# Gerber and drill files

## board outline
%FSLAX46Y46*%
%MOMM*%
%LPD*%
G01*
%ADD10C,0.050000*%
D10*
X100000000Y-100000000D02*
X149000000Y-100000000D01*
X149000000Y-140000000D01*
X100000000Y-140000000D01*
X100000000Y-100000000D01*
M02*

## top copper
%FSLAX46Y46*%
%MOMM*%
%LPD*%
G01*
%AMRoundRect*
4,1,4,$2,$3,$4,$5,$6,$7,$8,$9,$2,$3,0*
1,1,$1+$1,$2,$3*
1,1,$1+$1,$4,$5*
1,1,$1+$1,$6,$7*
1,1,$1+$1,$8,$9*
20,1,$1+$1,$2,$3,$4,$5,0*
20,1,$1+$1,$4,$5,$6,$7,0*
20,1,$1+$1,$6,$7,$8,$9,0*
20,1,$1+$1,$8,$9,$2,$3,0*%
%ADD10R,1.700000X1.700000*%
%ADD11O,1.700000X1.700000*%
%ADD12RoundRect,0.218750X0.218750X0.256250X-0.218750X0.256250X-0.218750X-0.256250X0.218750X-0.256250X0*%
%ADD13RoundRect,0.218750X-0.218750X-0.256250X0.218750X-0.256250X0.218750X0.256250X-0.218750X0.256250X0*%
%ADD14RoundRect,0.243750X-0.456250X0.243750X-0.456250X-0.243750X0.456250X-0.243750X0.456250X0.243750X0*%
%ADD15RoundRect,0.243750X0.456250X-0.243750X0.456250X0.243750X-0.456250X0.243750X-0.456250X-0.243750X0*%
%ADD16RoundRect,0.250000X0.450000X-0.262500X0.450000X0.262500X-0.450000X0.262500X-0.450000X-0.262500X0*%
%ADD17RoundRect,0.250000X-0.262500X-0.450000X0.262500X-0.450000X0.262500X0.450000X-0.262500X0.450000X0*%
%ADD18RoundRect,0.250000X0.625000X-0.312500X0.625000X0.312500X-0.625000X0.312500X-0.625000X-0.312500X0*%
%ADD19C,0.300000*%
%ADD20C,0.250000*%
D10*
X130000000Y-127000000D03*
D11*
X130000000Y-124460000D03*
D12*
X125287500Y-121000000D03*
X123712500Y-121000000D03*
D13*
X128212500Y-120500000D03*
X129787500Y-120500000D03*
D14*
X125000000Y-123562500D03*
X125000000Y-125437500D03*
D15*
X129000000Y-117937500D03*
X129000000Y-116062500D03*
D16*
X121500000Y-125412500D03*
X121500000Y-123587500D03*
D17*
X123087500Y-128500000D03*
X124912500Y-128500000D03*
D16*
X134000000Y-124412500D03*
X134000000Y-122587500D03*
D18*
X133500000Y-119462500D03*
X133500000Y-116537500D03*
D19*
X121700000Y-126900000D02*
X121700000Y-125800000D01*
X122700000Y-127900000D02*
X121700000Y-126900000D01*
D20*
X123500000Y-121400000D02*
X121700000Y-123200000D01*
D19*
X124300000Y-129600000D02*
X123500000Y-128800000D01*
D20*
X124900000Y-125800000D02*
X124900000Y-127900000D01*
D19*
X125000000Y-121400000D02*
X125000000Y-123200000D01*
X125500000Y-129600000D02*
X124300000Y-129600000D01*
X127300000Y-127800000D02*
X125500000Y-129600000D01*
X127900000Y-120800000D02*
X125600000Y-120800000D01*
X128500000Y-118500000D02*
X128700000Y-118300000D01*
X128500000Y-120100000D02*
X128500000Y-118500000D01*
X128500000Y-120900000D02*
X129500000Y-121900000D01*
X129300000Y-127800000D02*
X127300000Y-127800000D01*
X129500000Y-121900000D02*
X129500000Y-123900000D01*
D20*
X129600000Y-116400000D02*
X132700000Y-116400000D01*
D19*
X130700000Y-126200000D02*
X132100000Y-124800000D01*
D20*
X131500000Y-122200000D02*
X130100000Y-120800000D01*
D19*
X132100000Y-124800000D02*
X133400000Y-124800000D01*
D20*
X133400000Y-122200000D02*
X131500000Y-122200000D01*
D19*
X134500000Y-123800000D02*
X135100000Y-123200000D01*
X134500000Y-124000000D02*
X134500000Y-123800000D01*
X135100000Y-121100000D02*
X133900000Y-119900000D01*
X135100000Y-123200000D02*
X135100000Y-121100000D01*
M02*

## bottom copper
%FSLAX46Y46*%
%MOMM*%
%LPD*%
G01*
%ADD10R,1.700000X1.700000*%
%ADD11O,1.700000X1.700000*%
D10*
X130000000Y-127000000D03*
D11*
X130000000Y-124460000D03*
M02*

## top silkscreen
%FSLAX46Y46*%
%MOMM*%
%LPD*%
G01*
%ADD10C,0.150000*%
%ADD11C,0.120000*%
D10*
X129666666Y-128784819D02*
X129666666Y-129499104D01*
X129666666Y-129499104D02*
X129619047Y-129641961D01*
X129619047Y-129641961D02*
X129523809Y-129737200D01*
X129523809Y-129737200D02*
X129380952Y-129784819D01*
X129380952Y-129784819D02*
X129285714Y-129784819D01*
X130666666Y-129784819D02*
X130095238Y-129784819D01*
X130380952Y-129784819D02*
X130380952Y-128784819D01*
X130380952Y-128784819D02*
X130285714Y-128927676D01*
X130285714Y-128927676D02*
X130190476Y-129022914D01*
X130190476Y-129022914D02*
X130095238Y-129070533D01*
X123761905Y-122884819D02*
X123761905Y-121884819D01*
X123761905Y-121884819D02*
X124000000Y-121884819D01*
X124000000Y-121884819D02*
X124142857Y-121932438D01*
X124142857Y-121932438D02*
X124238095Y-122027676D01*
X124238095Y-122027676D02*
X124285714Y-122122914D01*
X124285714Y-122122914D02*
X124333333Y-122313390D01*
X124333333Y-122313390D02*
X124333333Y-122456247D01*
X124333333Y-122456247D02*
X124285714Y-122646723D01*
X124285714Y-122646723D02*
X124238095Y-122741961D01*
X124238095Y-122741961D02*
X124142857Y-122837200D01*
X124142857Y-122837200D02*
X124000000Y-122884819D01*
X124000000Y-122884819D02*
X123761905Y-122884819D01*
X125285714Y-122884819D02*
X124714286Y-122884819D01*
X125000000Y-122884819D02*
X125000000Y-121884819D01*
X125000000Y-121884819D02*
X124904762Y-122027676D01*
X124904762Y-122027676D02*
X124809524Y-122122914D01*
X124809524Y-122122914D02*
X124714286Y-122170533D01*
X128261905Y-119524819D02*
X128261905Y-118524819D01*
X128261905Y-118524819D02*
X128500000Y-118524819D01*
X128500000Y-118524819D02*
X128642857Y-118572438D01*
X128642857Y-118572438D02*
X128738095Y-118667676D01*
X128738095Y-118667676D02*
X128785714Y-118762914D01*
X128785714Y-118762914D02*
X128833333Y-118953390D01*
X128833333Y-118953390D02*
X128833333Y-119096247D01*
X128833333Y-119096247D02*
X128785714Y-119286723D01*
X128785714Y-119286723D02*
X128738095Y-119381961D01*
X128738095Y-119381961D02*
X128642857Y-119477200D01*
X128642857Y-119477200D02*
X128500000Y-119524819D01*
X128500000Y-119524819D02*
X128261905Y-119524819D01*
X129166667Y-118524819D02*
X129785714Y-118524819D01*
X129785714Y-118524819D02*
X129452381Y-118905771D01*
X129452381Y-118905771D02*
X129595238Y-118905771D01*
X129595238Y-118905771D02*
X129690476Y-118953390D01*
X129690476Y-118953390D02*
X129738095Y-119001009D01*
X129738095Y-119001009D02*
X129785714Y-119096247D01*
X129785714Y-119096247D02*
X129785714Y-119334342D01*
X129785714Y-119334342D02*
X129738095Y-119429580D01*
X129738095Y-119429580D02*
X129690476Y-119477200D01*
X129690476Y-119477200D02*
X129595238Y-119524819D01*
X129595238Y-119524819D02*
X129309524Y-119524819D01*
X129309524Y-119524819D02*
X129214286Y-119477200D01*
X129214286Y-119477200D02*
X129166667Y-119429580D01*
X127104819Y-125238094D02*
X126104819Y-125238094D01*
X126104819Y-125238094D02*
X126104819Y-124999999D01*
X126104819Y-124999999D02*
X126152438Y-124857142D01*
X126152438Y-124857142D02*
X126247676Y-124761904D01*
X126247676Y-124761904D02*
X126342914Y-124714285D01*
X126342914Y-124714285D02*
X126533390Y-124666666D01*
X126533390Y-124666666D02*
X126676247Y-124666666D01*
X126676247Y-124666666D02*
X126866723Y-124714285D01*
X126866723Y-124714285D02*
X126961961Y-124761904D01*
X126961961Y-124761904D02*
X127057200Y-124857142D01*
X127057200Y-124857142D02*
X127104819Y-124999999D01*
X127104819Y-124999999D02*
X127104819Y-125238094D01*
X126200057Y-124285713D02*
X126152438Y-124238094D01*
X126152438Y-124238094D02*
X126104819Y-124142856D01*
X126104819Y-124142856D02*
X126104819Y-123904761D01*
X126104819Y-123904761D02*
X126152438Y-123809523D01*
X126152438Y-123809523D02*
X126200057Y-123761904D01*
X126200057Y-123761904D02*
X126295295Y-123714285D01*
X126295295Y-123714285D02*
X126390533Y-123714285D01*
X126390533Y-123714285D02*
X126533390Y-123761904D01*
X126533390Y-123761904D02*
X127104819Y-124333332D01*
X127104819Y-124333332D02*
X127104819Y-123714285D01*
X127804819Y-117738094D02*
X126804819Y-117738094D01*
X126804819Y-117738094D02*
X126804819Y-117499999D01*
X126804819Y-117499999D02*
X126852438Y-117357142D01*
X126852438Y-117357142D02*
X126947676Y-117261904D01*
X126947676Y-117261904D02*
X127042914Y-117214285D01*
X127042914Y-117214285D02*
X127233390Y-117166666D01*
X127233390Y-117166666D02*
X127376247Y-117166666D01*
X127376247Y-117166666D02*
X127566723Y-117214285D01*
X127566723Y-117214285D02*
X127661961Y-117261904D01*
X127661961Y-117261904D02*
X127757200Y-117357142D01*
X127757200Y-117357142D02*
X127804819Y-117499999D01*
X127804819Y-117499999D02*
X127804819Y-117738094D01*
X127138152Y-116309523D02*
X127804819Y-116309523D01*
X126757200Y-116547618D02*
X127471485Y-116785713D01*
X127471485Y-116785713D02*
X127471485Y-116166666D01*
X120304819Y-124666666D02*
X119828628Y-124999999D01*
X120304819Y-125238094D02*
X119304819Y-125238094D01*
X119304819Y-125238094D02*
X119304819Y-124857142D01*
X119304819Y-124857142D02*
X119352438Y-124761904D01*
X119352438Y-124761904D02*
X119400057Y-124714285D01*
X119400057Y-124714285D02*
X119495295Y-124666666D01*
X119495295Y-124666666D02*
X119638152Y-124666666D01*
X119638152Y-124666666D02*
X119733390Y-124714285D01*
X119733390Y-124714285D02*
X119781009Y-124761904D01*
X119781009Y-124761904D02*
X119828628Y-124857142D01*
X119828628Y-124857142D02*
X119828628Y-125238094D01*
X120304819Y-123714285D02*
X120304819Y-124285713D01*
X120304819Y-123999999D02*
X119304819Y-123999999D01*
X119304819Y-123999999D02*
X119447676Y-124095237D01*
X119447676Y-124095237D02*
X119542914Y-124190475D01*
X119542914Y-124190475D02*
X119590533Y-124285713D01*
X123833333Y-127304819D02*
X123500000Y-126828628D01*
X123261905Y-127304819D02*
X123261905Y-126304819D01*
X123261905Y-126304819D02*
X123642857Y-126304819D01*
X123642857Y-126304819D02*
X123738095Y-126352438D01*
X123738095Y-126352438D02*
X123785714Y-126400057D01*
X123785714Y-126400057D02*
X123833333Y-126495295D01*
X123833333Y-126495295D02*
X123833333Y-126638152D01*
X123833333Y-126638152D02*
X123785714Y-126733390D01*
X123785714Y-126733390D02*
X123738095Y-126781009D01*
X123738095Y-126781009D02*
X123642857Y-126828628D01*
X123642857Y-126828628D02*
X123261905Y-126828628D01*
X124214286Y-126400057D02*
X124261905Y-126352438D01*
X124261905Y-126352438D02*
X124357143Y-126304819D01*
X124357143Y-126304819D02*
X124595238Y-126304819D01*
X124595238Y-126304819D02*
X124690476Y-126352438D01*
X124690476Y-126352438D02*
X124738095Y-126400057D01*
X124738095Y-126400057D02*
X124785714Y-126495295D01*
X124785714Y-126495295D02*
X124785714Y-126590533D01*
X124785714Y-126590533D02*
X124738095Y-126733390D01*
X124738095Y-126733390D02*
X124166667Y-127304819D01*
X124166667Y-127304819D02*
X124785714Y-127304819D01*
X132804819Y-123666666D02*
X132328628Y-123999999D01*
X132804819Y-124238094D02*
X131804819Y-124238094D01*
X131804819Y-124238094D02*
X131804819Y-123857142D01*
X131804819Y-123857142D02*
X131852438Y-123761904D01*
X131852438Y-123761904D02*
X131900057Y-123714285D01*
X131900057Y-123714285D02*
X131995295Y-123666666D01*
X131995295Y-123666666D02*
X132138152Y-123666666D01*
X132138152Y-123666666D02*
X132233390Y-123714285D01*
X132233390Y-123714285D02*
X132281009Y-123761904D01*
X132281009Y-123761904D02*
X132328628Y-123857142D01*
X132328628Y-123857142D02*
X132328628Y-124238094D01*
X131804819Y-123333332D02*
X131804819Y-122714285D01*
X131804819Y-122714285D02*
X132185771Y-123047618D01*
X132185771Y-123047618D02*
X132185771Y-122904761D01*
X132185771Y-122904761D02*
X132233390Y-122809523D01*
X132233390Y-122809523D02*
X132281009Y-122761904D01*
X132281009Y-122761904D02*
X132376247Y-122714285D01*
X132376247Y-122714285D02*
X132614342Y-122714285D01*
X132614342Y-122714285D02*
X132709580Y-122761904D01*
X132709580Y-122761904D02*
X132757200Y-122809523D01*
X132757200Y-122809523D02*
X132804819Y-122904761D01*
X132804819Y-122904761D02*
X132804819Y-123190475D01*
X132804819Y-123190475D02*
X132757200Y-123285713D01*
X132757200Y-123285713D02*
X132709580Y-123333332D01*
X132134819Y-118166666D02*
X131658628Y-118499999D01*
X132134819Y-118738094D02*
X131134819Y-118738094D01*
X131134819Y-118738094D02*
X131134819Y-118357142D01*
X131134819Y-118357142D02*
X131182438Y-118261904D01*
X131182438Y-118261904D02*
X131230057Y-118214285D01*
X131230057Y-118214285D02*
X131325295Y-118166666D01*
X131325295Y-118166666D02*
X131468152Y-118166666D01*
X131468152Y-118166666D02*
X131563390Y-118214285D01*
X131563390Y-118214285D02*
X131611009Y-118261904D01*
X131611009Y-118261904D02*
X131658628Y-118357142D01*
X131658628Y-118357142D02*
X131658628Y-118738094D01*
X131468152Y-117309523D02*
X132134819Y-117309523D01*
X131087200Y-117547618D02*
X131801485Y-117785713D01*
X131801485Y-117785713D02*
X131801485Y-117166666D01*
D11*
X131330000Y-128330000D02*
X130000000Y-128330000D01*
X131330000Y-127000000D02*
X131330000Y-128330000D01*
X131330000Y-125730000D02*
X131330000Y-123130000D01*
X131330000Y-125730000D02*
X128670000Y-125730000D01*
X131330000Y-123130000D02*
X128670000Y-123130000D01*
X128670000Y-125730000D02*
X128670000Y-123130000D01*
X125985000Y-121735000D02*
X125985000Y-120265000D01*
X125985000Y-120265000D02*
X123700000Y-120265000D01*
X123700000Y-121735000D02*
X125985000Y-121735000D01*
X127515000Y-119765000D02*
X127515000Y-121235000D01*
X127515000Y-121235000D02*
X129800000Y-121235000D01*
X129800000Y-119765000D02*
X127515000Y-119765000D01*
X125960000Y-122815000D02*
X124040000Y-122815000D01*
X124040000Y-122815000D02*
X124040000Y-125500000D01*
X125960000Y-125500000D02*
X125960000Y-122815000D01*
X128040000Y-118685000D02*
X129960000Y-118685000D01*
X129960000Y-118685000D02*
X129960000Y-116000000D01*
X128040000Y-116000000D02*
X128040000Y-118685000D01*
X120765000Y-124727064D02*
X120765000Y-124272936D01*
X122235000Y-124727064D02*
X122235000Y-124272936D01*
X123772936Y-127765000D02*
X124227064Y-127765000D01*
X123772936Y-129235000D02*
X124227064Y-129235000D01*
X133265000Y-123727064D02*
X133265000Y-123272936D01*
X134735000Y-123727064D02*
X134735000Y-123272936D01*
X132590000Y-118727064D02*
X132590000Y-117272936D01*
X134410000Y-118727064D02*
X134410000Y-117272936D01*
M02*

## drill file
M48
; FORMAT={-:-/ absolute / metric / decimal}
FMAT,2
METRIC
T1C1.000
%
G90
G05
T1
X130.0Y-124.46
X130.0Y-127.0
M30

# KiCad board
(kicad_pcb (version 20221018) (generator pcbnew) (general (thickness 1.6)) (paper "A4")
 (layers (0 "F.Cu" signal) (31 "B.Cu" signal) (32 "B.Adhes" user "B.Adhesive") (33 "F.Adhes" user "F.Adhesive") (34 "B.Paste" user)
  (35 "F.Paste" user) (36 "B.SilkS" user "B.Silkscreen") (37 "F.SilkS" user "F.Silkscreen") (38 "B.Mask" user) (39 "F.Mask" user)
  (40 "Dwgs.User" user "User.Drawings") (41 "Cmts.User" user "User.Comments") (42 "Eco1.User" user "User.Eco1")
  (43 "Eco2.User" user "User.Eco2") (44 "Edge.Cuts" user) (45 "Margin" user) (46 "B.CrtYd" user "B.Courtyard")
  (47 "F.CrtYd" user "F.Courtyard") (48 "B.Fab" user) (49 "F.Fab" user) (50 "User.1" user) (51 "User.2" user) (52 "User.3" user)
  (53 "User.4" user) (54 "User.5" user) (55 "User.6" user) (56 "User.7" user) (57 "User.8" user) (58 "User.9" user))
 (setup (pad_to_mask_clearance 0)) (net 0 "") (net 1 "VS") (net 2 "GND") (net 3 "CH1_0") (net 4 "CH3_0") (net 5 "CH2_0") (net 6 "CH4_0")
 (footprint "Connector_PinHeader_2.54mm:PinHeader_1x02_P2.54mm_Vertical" (layer "F.Cu") (at 130 127 180)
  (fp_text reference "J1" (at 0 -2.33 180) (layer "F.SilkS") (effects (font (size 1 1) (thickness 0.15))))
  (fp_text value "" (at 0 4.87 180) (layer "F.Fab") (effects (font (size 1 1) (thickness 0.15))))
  (fp_line (start -1.33 -1.33) (end 0 -1.33) (stroke (width 0.12) (type solid)) (layer "F.SilkS"))
  (fp_line (start -1.33 0) (end -1.33 -1.33) (stroke (width 0.12) (type solid)) (layer "F.SilkS"))
  (fp_line (start -1.33 1.27) (end -1.33 3.87) (stroke (width 0.12) (type solid)) (layer "F.SilkS"))
  (fp_line (start -1.33 1.27) (end 1.33 1.27) (stroke (width 0.12) (type solid)) (layer "F.SilkS"))
  (fp_line (start -1.33 3.87) (end 1.33 3.87) (stroke (width 0.12) (type solid)) (layer "F.SilkS"))
  (fp_line (start 1.33 1.27) (end 1.33 3.87) (stroke (width 0.12) (type solid)) (layer "F.SilkS"))
  (pad "1" thru_hole rect (at 0 0 180) (size 1.7 1.7) (drill 1) (layers "*.Cu" "*.Mask") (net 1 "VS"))
  (pad "2" thru_hole oval (at 0 2.54 180) (size 1.7 1.7) (drill 1) (layers "*.Cu" "*.Mask") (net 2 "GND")))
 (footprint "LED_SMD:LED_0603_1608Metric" (layer "F.Cu") (at 124.5 121 180)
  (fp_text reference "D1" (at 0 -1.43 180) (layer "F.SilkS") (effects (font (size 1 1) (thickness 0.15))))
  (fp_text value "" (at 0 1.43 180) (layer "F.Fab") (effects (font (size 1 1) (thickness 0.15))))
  (fp_line (start -1.485 -0.735) (end -1.485 0.735) (stroke (width 0.12) (type solid)) (layer "F.SilkS"))
  (fp_line (start -1.485 0.735) (end 0.8 0.735) (stroke (width 0.12) (type solid)) (layer "F.SilkS"))
  (fp_line (start 0.8 -0.735) (end -1.485 -0.735) (stroke (width 0.12) (type solid)) (layer "F.SilkS"))
  (pad "1" smd roundrect (at -0.7875 0 180) (size 0.875 0.95) (layers "F.Cu" "F.Paste" "F.Mask") (roundrect_rratio 0.25) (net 2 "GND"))
  (pad "2" smd roundrect (at 0.7875 0 180) (size 0.875 0.95) (layers "F.Cu" "F.Paste" "F.Mask") (roundrect_rratio 0.25) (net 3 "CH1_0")))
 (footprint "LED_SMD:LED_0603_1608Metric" (layer "F.Cu") (at 129 120.5)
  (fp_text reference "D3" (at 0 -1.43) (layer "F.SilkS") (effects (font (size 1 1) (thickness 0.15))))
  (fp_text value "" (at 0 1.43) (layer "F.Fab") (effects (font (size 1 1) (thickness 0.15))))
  (fp_line (start -1.485 -0.735) (end -1.485 0.735) (stroke (width 0.12) (type solid)) (layer "F.SilkS"))
  (fp_line (start -1.485 0.735) (end 0.8 0.735) (stroke (width 0.12) (type solid)) (layer "F.SilkS"))
  (fp_line (start 0.8 -0.735) (end -1.485 -0.735) (stroke (width 0.12) (type solid)) (layer "F.SilkS"))
  (pad "1" smd roundrect (at -0.7875 0) (size 0.875 0.95) (layers "F.Cu" "F.Paste" "F.Mask") (roundrect_rratio 0.25) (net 2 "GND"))
  (pad "2" smd roundrect (at 0.7875 0) (size 0.875 0.95) (layers "F.Cu" "F.Paste" "F.Mask") (roundrect_rratio 0.25) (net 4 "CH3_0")))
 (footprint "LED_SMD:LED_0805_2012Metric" (layer "F.Cu") (at 125 124.5 -90)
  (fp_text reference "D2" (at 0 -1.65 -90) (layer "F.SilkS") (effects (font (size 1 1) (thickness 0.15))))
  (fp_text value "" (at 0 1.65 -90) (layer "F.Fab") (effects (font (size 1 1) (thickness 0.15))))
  (fp_line (start -1.685 -0.96) (end -1.685 0.96) (stroke (width 0.12) (type solid)) (layer "F.SilkS"))
  (fp_line (start -1.685 0.96) (end 1 0.96) (stroke (width 0.12) (type solid)) (layer "F.SilkS"))
  (fp_line (start 1 -0.96) (end -1.685 -0.96) (stroke (width 0.12) (type solid)) (layer "F.SilkS"))
  (pad "1" smd roundrect (at -0.9375 0 270) (size 0.975 1.4) (layers "F.Cu" "F.Paste" "F.Mask") (roundrect_rratio 0.25) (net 2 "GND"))
  (pad "2" smd roundrect (at 0.9375 0 270) (size 0.975 1.4) (layers "F.Cu" "F.Paste" "F.Mask") (roundrect_rratio 0.25) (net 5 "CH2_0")))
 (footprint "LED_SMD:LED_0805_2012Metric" (layer "F.Cu") (at 129 117 90)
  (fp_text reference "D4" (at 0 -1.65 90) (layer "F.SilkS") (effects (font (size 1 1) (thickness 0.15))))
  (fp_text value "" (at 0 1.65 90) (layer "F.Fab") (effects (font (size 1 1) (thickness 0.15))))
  (fp_line (start -1.685 -0.96) (end -1.685 0.96) (stroke (width 0.12) (type solid)) (layer "F.SilkS"))
  (fp_line (start -1.685 0.96) (end 1 0.96) (stroke (width 0.12) (type solid)) (layer "F.SilkS"))
  (fp_line (start 1 -0.96) (end -1.685 -0.96) (stroke (width 0.12) (type solid)) (layer "F.SilkS"))
  (pad "1" smd roundrect (at -0.9375 0 90) (size 0.975 1.4) (layers "F.Cu" "F.Paste" "F.Mask") (roundrect_rratio 0.25) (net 2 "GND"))
  (pad "2" smd roundrect (at 0.9375 0 90) (size 0.975 1.4) (layers "F.Cu" "F.Paste" "F.Mask") (roundrect_rratio 0.25) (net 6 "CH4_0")))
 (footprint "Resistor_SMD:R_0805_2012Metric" (layer "F.Cu") (at 121.5 124.5 90)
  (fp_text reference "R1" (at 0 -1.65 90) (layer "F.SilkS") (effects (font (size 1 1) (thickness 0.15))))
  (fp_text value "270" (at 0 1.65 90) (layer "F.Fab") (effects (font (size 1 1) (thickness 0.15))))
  (fp_line (start -0.227064 -0.735) (end 0.227064 -0.735) (stroke (width 0.12) (type solid)) (layer "F.SilkS"))
  (fp_line (start -0.227064 0.735) (end 0.227064 0.735) (stroke (width 0.12) (type solid)) (layer "F.SilkS"))
  (pad "1" smd roundrect (at -0.9125 0 90) (size 1.025 1.4) (layers "F.Cu" "F.Paste" "F.Mask") (roundrect_rratio 0.243902) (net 1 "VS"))
  (pad "2" smd roundrect (at 0.9125 0 90) (size 1.025 1.4) (layers "F.Cu" "F.Paste" "F.Mask") (roundrect_rratio 0.243902) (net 3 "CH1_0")))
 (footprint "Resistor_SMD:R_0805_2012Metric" (layer "F.Cu") (at 124 128.5)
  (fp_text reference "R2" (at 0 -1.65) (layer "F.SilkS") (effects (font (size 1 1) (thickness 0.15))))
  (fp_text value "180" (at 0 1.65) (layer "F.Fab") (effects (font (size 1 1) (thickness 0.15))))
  (fp_line (start -0.227064 -0.735) (end 0.227064 -0.735) (stroke (width 0.12) (type solid)) (layer "F.SilkS"))
  (fp_line (start -0.227064 0.735) (end 0.227064 0.735) (stroke (width 0.12) (type solid)) (layer "F.SilkS"))
  (pad "1" smd roundrect (at -0.9125 0) (size 1.025 1.4) (layers "F.Cu" "F.Paste" "F.Mask") (roundrect_rratio 0.243902) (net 1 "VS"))
  (pad "2" smd roundrect (at 0.9125 0) (size 1.025 1.4) (layers "F.Cu" "F.Paste" "F.Mask") (roundrect_rratio 0.243902) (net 5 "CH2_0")))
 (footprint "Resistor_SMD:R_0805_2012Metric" (layer "F.Cu") (at 134 123.5 90)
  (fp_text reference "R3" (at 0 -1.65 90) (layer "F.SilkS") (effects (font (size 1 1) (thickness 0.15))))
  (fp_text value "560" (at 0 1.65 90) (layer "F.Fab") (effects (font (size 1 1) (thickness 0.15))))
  (fp_line (start -0.227064 -0.735) (end 0.227064 -0.735) (stroke (width 0.12) (type solid)) (layer "F.SilkS"))
  (fp_line (start -0.227064 0.735) (end 0.227064 0.735) (stroke (width 0.12) (type solid)) (layer "F.SilkS"))
  (pad "1" smd roundrect (at -0.9125 0 90) (size 1.025 1.4) (layers "F.Cu" "F.Paste" "F.Mask") (roundrect_rratio 0.243902) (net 1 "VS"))
  (pad "2" smd roundrect (at 0.9125 0 90) (size 1.025 1.4) (layers "F.Cu" "F.Paste" "F.Mask") (roundrect_rratio 0.243902) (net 4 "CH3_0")))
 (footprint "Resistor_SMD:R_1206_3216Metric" (layer "F.Cu") (at 133.5 118 90)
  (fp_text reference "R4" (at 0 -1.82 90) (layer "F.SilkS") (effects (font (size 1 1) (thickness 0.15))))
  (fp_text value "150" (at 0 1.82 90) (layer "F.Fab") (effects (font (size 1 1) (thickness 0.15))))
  (fp_line (start -0.727064 -0.91) (end 0.727064 -0.91) (stroke (width 0.12) (type solid)) (layer "F.SilkS"))
  (fp_line (start -0.727064 0.91) (end 0.727064 0.91) (stroke (width 0.12) (type solid)) (layer "F.SilkS"))
  (pad "1" smd roundrect (at -1.4625 0 90) (size 1.125 1.75) (layers "F.Cu" "F.Paste" "F.Mask") (roundrect_rratio 0.222222) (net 1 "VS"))
  (pad "2" smd roundrect (at 1.4625 0 90) (size 1.125 1.75) (layers "F.Cu" "F.Paste" "F.Mask") (roundrect_rratio 0.222222) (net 6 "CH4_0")))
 (gr_rect (start 100 100) (end 149 140) (stroke (width 0.05) (type default)) (fill none) (layer "Edge.Cuts"))
 (segment (start 121.7 126.9) (end 121.7 125.8) (width 0.3) (layer "F.Cu") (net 1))
 (segment (start 122.7 127.9) (end 121.7 126.9) (width 0.3) (layer "F.Cu") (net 1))
 (segment (start 123.5 121.4) (end 121.7 123.2) (width 0.25) (layer "F.Cu") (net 3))
 (segment (start 124.3 129.6) (end 123.5 128.8) (width 0.3) (layer "F.Cu") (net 1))
 (segment (start 124.9 125.8) (end 124.9 127.9) (width 0.25) (layer "F.Cu") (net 5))
 (segment (start 125 121.4) (end 125 123.2) (width 0.3) (layer "F.Cu") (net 2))
 (segment (start 125.5 129.6) (end 124.3 129.6) (width 0.3) (layer "F.Cu") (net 1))
 (segment (start 127.3 127.8) (end 125.5 129.6) (width 0.3) (layer "F.Cu") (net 1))
 (segment (start 127.9 120.8) (end 125.6 120.8) (width 0.3) (layer "F.Cu") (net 2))
 (segment (start 128.5 118.5) (end 128.7 118.3) (width 0.3) (layer "F.Cu") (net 2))
 (segment (start 128.5 120.1) (end 128.5 118.5) (width 0.3) (layer "F.Cu") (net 2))
 (segment (start 128.5 120.9) (end 129.5 121.9) (width 0.3) (layer "F.Cu") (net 2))
 (segment (start 129.3 127.8) (end 127.3 127.8) (width 0.3) (layer "F.Cu") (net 1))
 (segment (start 129.5 121.9) (end 129.5 123.9) (width 0.3) (layer "F.Cu") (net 2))
 (segment (start 129.6 116.4) (end 132.7 116.4) (width 0.25) (layer "F.Cu") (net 6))
 (segment (start 130.7 126.2) (end 132.1 124.8) (width 0.3) (layer "F.Cu") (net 1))
 (segment (start 131.5 122.2) (end 130.1 120.8) (width 0.25) (layer "F.Cu") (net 4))
 (segment (start 132.1 124.8) (end 133.4 124.8) (width 0.3) (layer "F.Cu") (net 1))
 (segment (start 133.4 122.2) (end 131.5 122.2) (width 0.25) (layer "F.Cu") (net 4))
 (segment (start 134.5 123.8) (end 135.1 123.2) (width 0.3) (layer "F.Cu") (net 1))
 (segment (start 134.5 124) (end 134.5 123.8) (width 0.3) (layer "F.Cu") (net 1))
 (segment (start 135.1 121.1) (end 133.9 119.9) (width 0.3) (layer "F.Cu") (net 1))
 (segment (start 135.1 123.2) (end 135.1 121.1) (width 0.3) (layer "F.Cu") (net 1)))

